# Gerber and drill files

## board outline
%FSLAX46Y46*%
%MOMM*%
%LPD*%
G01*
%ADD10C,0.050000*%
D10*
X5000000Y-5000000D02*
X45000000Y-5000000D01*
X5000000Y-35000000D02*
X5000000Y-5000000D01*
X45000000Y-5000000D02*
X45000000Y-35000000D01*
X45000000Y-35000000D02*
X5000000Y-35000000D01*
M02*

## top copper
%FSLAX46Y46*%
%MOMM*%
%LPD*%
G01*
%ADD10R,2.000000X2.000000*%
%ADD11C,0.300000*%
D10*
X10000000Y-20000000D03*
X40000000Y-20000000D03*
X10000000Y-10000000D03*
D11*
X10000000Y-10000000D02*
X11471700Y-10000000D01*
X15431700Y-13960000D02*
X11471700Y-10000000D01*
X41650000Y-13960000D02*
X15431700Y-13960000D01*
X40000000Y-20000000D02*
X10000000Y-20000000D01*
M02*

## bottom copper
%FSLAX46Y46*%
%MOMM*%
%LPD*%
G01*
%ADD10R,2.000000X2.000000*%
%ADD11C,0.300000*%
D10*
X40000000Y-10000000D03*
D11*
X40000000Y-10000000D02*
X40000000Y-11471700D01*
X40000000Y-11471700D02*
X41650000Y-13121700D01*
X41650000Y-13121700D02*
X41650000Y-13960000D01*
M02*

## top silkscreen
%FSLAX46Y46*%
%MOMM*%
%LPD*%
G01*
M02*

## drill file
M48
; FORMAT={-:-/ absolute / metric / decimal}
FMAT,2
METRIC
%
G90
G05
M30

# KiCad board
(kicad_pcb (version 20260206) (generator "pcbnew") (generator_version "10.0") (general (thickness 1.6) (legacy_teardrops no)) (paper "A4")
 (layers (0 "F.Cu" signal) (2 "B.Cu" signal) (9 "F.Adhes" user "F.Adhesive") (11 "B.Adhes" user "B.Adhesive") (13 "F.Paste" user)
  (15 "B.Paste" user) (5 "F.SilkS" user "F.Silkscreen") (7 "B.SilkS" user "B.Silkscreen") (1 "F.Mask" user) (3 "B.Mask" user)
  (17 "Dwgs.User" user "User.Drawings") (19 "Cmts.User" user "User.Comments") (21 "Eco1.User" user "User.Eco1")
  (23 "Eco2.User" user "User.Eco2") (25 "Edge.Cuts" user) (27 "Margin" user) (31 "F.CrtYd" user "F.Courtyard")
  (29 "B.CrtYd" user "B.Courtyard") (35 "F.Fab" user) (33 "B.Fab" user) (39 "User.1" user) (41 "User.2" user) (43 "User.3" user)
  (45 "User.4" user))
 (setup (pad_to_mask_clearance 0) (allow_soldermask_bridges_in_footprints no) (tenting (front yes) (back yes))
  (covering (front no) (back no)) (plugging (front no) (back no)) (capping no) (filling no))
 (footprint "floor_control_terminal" (layer "F.Cu") (at 10 20)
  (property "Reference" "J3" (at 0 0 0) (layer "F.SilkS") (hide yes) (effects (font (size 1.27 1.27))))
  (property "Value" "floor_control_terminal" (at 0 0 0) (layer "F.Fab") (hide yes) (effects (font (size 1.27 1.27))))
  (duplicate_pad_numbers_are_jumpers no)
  (pad "1" smd rect (at 0 0) (size 2 2) (layers "F.Cu" "F.Mask" "F.Paste") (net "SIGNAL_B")))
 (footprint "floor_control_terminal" (layer "F.Cu") (at 40 20)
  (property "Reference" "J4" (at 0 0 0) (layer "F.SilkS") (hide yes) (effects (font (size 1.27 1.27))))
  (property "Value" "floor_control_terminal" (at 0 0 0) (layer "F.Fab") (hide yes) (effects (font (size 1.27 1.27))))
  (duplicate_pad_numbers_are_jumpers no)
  (pad "1" smd rect (at 0 0) (size 2 2) (layers "F.Cu" "F.Mask" "F.Paste") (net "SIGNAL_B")))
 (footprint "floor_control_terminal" (layer "F.Cu") (at 10 10)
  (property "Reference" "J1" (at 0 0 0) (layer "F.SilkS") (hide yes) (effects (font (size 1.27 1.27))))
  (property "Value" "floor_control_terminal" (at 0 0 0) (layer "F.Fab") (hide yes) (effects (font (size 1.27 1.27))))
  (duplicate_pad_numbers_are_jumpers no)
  (pad "1" smd rect (at 0 0) (size 2 2) (layers "F.Cu" "F.Mask" "F.Paste") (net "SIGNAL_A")))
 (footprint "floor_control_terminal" (layer "B.Cu") (at 40 10)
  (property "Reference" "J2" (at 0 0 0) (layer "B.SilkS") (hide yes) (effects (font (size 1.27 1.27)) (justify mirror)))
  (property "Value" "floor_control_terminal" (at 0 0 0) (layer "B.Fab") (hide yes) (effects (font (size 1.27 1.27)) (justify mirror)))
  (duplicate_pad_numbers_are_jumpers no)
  (pad "1" smd rect (at 0 0) (size 2 2) (layers "B.Cu" "B.Mask" "B.Paste") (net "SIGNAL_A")))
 (gr_line (start 5 5) (end 45 5) (stroke (width 0.05) (type default)) (layer "Edge.Cuts"))
 (gr_line (start 5 35) (end 5 5) (stroke (width 0.05) (type default)) (layer "Edge.Cuts"))
 (gr_line (start 45 5) (end 45 35) (stroke (width 0.05) (type default)) (layer "Edge.Cuts"))
 (gr_line (start 45 35) (end 5 35) (stroke (width 0.05) (type default)) (layer "Edge.Cuts"))
 (segment (start 10 10) (end 11.4717 10) (width 0.3) (layer "F.Cu") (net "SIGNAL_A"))
 (segment (start 15.4317 13.96) (end 11.4717 10) (width 0.3) (layer "F.Cu") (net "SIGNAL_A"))
 (segment (start 41.65 13.96) (end 15.4317 13.96) (width 0.3) (layer "F.Cu") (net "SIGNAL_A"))
 (segment (start 40 10) (end 40 11.4717) (width 0.3) (layer "B.Cu") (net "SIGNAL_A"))
 (segment (start 40 11.4717) (end 41.65 13.1217) (width 0.3) (layer "B.Cu") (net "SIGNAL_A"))
 (segment (start 41.65 13.1217) (end 41.65 13.96) (width 0.3) (layer "B.Cu") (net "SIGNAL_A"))
 (segment (start 40 20) (end 10 20) (width 0.3) (layer "F.Cu") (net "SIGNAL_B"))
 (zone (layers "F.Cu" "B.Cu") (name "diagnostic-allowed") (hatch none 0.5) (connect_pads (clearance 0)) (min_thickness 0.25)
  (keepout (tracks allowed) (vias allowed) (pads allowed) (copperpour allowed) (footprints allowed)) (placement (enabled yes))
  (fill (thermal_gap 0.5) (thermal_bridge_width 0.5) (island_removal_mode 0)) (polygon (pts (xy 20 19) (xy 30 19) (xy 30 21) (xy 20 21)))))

